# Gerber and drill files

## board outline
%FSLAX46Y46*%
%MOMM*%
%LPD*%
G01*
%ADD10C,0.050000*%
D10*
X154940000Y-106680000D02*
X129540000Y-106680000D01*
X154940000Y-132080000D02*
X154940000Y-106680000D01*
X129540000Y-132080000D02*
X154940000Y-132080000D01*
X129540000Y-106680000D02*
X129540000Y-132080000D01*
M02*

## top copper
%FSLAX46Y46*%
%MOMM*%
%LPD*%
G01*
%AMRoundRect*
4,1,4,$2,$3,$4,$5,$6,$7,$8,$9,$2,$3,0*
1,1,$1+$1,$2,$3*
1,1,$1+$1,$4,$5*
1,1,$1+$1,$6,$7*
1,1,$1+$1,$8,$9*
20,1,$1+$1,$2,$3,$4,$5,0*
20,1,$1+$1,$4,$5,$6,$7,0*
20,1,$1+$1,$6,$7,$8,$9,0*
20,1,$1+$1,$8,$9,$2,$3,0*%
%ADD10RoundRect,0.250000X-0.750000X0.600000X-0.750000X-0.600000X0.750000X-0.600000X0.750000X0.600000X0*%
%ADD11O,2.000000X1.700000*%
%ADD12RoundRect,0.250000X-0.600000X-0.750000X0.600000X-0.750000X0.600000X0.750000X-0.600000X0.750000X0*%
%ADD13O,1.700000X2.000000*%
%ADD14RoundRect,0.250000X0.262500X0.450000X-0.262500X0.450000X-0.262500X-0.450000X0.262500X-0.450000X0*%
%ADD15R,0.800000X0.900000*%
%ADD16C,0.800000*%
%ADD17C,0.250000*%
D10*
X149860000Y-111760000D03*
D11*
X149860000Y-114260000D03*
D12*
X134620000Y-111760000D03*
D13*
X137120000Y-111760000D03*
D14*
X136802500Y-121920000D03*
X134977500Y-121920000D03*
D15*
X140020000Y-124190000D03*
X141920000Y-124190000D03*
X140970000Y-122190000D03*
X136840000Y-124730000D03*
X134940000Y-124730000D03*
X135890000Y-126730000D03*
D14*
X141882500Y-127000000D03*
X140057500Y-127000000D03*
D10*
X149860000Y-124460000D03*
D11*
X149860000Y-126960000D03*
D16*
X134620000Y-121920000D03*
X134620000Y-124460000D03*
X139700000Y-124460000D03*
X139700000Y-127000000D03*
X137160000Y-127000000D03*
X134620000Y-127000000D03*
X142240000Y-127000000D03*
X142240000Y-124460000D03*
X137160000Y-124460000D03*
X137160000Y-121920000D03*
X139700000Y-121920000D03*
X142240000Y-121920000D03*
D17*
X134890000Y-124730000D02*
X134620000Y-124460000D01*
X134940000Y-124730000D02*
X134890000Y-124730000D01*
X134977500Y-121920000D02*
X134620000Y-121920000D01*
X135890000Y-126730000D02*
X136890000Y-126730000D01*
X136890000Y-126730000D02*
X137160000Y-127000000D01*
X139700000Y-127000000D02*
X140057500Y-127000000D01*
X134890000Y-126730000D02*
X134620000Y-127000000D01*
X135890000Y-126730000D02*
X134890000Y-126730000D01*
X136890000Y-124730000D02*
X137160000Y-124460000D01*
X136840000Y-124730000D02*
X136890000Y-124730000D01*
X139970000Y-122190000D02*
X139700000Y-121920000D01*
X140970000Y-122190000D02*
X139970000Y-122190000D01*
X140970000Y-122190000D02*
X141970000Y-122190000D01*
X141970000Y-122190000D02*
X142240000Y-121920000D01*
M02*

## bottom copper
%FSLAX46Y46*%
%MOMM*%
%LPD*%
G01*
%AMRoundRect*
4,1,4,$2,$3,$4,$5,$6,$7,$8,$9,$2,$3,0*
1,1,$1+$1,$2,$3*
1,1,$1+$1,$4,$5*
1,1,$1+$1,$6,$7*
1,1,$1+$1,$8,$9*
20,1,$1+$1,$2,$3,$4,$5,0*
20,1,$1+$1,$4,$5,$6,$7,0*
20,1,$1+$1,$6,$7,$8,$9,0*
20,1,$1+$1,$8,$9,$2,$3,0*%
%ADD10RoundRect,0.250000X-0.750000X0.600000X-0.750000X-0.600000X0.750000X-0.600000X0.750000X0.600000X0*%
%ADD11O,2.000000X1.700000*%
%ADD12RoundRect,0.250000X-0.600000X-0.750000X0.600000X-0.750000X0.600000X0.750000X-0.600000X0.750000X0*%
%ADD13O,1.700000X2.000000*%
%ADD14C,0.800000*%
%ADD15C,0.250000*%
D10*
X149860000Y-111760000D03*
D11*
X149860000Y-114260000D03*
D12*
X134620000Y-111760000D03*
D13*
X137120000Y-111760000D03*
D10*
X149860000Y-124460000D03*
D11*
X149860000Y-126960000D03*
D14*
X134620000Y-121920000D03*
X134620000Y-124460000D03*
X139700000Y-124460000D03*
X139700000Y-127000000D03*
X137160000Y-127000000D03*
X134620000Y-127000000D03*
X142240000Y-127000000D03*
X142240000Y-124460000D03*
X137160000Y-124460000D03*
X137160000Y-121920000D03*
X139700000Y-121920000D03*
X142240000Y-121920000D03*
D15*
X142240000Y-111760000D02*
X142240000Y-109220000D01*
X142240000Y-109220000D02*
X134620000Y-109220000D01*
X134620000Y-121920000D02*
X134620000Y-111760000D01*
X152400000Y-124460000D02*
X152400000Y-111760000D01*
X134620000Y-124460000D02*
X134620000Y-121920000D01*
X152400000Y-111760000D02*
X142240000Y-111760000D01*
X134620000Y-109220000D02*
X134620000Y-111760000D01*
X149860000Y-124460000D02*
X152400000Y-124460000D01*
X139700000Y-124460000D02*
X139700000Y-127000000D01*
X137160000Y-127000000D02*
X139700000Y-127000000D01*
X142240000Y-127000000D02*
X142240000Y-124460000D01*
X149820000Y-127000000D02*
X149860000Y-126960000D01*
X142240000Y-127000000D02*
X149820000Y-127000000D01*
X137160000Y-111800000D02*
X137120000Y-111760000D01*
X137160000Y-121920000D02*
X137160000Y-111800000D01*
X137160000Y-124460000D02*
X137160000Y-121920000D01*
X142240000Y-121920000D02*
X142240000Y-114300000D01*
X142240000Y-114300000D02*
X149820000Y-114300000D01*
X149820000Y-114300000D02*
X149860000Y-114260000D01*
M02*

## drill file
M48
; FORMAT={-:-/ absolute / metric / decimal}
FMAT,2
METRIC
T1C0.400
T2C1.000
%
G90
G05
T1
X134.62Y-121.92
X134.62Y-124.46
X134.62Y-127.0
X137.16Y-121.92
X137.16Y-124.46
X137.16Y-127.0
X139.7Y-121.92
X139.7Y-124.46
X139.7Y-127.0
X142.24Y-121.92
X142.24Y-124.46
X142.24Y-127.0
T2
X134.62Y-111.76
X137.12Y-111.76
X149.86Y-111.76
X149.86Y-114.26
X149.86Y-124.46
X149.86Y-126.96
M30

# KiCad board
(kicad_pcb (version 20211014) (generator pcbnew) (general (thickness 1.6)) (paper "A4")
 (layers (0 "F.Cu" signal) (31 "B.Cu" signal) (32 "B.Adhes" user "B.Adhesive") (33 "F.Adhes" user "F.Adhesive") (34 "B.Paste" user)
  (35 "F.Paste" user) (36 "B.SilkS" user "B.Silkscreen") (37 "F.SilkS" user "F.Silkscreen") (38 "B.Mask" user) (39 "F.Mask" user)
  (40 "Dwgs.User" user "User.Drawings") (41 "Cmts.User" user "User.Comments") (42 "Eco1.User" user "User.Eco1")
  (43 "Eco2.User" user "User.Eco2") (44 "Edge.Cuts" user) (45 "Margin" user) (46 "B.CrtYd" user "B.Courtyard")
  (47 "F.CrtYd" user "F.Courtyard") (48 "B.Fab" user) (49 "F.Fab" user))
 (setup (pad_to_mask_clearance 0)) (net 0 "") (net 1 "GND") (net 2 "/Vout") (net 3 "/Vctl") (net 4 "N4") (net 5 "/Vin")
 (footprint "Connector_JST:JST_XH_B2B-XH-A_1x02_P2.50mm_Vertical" (layer "F.Cu") (at 149.86 111.76 -90)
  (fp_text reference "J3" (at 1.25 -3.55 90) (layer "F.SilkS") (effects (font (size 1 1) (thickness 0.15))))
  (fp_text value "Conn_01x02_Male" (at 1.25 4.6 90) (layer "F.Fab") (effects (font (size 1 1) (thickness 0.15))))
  (pad "1" thru_hole roundrect locked (at 0 0 270) (size 1.7 2) (drill 1) (layers *.Cu *.Mask) (roundrect_rratio 0.147059) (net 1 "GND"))
  (pad "2" thru_hole oval locked (at 2.5 0 270) (size 1.7 2) (drill 1) (layers *.Cu *.Mask) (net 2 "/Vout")))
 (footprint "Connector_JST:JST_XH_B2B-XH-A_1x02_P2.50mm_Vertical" (layer "F.Cu") (at 134.62 111.76)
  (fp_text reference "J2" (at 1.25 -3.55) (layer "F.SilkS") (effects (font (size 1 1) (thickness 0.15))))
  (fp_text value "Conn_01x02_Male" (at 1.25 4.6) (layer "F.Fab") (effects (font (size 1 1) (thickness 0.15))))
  (pad "1" thru_hole roundrect locked (at 0 0) (size 1.7 2) (drill 1) (layers *.Cu *.Mask) (roundrect_rratio 0.147059) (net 1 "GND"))
  (pad "2" thru_hole oval locked (at 2.5 0) (size 1.7 2) (drill 1) (layers *.Cu *.Mask) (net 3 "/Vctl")))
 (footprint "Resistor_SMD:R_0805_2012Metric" (layer "F.Cu") (at 135.89 121.92 180)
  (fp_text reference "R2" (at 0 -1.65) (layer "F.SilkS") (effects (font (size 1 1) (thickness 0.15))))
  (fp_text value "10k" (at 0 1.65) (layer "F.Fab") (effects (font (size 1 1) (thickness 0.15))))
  (pad "1" smd roundrect locked (at -0.9125 0 180) (size 1.025 1.4) (layers "F.Cu" "F.Paste" "F.Mask") (roundrect_rratio 0.243902)
   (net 3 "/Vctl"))
  (pad "2" smd roundrect locked (at 0.9125 0 180) (size 1.025 1.4) (layers "F.Cu" "F.Paste" "F.Mask") (roundrect_rratio 0.243902)
   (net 1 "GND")))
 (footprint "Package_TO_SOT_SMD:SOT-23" (layer "F.Cu") (at 140.97 123.19 90)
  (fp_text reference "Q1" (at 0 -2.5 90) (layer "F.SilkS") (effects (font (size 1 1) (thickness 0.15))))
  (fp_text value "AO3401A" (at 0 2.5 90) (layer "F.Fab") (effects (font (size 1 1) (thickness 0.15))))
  (pad "1" smd rect locked (at -1 -0.95 90) (size 0.9 0.8) (layers "F.Cu" "F.Paste" "F.Mask") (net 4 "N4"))
  (pad "2" smd rect locked (at -1 0.95 90) (size 0.9 0.8) (layers "F.Cu" "F.Paste" "F.Mask") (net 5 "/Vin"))
  (pad "3" smd rect locked (at 1 0 90) (size 0.9 0.8) (layers "F.Cu" "F.Paste" "F.Mask") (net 2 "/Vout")))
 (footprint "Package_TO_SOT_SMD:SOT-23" (layer "F.Cu") (at 135.89 125.73 -90)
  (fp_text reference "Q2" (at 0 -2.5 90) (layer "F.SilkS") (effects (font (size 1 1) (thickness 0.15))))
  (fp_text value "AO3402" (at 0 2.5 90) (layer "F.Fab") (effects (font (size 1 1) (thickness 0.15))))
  (pad "1" smd rect locked (at -1 -0.95 270) (size 0.9 0.8) (layers "F.Cu" "F.Paste" "F.Mask") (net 3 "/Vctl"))
  (pad "2" smd rect locked (at -1 0.95 270) (size 0.9 0.8) (layers "F.Cu" "F.Paste" "F.Mask") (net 1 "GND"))
  (pad "3" smd rect locked (at 1 0 270) (size 0.9 0.8) (layers "F.Cu" "F.Paste" "F.Mask") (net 4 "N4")))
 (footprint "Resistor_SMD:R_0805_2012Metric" (layer "F.Cu") (at 140.97 127 180)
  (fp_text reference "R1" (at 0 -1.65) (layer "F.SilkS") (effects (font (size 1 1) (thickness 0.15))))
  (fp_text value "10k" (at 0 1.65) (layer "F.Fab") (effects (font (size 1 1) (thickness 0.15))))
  (pad "1" smd roundrect locked (at -0.9125 0 180) (size 1.025 1.4) (layers "F.Cu" "F.Paste" "F.Mask") (roundrect_rratio 0.243902)
   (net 5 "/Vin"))
  (pad "2" smd roundrect locked (at 0.9125 0 180) (size 1.025 1.4) (layers "F.Cu" "F.Paste" "F.Mask") (roundrect_rratio 0.243902)
   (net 4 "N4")))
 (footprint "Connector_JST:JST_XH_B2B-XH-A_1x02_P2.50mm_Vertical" (layer "F.Cu") (at 149.86 124.46 -90)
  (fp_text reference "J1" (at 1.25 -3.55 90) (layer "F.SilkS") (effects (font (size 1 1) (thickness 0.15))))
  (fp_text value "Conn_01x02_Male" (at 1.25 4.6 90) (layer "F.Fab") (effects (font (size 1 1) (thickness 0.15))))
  (pad "1" thru_hole roundrect locked (at 0 0 270) (size 1.7 2) (drill 1) (layers *.Cu *.Mask) (roundrect_rratio 0.147059) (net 1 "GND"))
  (pad "2" thru_hole oval locked (at 2.5 0 270) (size 1.7 2) (drill 1) (layers *.Cu *.Mask) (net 5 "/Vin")))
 (gr_line (start 154.94 106.68) (end 129.54 106.68) (layer "Edge.Cuts") (width 0.05))
 (gr_line (start 154.94 132.08) (end 154.94 106.68) (layer "Edge.Cuts") (width 0.05))
 (gr_line (start 129.54 132.08) (end 154.94 132.08) (layer "Edge.Cuts") (width 0.05))
 (gr_line (start 129.54 106.68) (end 129.54 132.08) (layer "Edge.Cuts") (width 0.05))
 (segment (start 134.89 124.73) (end 134.62 124.46) (width 0.25) (layer "F.Cu") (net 1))
 (segment (start 134.94 124.73) (end 134.89 124.73) (width 0.25) (layer "F.Cu") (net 1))
 (segment (start 134.9775 121.92) (end 134.62 121.92) (width 0.25) (layer "F.Cu") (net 1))
 (via (at 134.62 121.92) (size 0.8) (drill 0.4) (layers "F.Cu" "B.Cu") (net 1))
 (via (at 134.62 124.46) (size 0.8) (drill 0.4) (layers "F.Cu" "B.Cu") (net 1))
 (segment (start 142.24 111.76) (end 142.24 109.22) (width 0.25) (layer "B.Cu") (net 1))
 (segment (start 142.24 109.22) (end 134.62 109.22) (width 0.25) (layer "B.Cu") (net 1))
 (segment (start 134.62 121.92) (end 134.62 111.76) (width 0.25) (layer "B.Cu") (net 1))
 (segment (start 152.4 124.46) (end 152.4 111.76) (width 0.25) (layer "B.Cu") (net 1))
 (segment (start 134.62 124.46) (end 134.62 121.92) (width 0.25) (layer "B.Cu") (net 1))
 (segment (start 152.4 111.76) (end 142.24 111.76) (width 0.25) (layer "B.Cu") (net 1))
 (segment (start 134.62 109.22) (end 134.62 111.76) (width 0.25) (layer "B.Cu") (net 1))
 (segment (start 149.86 124.46) (end 152.4 124.46) (width 0.25) (layer "B.Cu") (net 1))
 (segment (start 135.89 126.73) (end 136.89 126.73) (width 0.25) (layer "F.Cu") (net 4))
 (segment (start 136.89 126.73) (end 137.16 127) (width 0.25) (layer "F.Cu") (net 4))
 (segment (start 139.7 127) (end 140.0575 127) (width 0.25) (layer "F.Cu") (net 4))
 (segment (start 134.89 126.73) (end 134.62 127) (width 0.25) (layer "F.Cu") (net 4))
 (segment (start 135.89 126.73) (end 134.89 126.73) (width 0.25) (layer "F.Cu") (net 4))
 (via (at 139.7 124.46) (size 0.8) (drill 0.4) (layers "F.Cu" "B.Cu") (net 4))
 (via (at 139.7 127) (size 0.8) (drill 0.4) (layers "F.Cu" "B.Cu") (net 4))
 (via (at 137.16 127) (size 0.8) (drill 0.4) (layers "F.Cu" "B.Cu") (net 4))
 (via (at 134.62 127) (size 0.8) (drill 0.4) (layers "F.Cu" "B.Cu") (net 4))
 (segment (start 139.7 124.46) (end 139.7 127) (width 0.25) (layer "B.Cu") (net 4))
 (segment (start 137.16 127) (end 139.7 127) (width 0.25) (layer "B.Cu") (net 4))
 (via (at 142.24 127) (size 0.8) (drill 0.4) (layers "F.Cu" "B.Cu") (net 5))
 (via (at 142.24 124.46) (size 0.8) (drill 0.4) (layers "F.Cu" "B.Cu") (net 5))
 (segment (start 142.24 127) (end 142.24 124.46) (width 0.25) (layer "B.Cu") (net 5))
 (segment (start 149.82 127) (end 149.86 126.96) (width 0.25) (layer "B.Cu") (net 5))
 (segment (start 142.24 127) (end 149.82 127) (width 0.25) (layer "B.Cu") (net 5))
 (segment (start 136.89 124.73) (end 137.16 124.46) (width 0.25) (layer "F.Cu") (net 3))
 (segment (start 136.84 124.73) (end 136.89 124.73) (width 0.25) (layer "F.Cu") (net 3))
 (via (at 137.16 124.46) (size 0.8) (drill 0.4) (layers "F.Cu" "B.Cu") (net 3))
 (via (at 137.16 121.92) (size 0.8) (drill 0.4) (layers "F.Cu" "B.Cu") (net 3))
 (segment (start 137.16 111.8) (end 137.12 111.76) (width 0.25) (layer "B.Cu") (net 3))
 (segment (start 137.16 121.92) (end 137.16 111.8) (width 0.25) (layer "B.Cu") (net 3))
 (segment (start 137.16 124.46) (end 137.16 121.92) (width 0.25) (layer "B.Cu") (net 3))
 (segment (start 139.97 122.19) (end 139.7 121.92) (width 0.25) (layer "F.Cu") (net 2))
 (segment (start 140.97 122.19) (end 139.97 122.19) (width 0.25) (layer "F.Cu") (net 2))
 (segment (start 140.97 122.19) (end 141.97 122.19) (width 0.25) (layer "F.Cu") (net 2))
 (segment (start 141.97 122.19) (end 142.24 121.92) (width 0.25) (layer "F.Cu") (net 2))
 (via (at 139.7 121.92) (size 0.8) (drill 0.4) (layers "F.Cu" "B.Cu") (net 2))
 (via (at 142.24 121.92) (size 0.8) (drill 0.4) (layers "F.Cu" "B.Cu") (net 2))
 (segment (start 142.24 121.92) (end 142.24 114.3) (width 0.25) (layer "B.Cu") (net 2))
 (segment (start 142.24 114.3) (end 149.82 114.3) (width 0.25) (layer "B.Cu") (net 2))
 (segment (start 149.82 114.3) (end 149.86 114.26) (width 0.25) (layer "B.Cu") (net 2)))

